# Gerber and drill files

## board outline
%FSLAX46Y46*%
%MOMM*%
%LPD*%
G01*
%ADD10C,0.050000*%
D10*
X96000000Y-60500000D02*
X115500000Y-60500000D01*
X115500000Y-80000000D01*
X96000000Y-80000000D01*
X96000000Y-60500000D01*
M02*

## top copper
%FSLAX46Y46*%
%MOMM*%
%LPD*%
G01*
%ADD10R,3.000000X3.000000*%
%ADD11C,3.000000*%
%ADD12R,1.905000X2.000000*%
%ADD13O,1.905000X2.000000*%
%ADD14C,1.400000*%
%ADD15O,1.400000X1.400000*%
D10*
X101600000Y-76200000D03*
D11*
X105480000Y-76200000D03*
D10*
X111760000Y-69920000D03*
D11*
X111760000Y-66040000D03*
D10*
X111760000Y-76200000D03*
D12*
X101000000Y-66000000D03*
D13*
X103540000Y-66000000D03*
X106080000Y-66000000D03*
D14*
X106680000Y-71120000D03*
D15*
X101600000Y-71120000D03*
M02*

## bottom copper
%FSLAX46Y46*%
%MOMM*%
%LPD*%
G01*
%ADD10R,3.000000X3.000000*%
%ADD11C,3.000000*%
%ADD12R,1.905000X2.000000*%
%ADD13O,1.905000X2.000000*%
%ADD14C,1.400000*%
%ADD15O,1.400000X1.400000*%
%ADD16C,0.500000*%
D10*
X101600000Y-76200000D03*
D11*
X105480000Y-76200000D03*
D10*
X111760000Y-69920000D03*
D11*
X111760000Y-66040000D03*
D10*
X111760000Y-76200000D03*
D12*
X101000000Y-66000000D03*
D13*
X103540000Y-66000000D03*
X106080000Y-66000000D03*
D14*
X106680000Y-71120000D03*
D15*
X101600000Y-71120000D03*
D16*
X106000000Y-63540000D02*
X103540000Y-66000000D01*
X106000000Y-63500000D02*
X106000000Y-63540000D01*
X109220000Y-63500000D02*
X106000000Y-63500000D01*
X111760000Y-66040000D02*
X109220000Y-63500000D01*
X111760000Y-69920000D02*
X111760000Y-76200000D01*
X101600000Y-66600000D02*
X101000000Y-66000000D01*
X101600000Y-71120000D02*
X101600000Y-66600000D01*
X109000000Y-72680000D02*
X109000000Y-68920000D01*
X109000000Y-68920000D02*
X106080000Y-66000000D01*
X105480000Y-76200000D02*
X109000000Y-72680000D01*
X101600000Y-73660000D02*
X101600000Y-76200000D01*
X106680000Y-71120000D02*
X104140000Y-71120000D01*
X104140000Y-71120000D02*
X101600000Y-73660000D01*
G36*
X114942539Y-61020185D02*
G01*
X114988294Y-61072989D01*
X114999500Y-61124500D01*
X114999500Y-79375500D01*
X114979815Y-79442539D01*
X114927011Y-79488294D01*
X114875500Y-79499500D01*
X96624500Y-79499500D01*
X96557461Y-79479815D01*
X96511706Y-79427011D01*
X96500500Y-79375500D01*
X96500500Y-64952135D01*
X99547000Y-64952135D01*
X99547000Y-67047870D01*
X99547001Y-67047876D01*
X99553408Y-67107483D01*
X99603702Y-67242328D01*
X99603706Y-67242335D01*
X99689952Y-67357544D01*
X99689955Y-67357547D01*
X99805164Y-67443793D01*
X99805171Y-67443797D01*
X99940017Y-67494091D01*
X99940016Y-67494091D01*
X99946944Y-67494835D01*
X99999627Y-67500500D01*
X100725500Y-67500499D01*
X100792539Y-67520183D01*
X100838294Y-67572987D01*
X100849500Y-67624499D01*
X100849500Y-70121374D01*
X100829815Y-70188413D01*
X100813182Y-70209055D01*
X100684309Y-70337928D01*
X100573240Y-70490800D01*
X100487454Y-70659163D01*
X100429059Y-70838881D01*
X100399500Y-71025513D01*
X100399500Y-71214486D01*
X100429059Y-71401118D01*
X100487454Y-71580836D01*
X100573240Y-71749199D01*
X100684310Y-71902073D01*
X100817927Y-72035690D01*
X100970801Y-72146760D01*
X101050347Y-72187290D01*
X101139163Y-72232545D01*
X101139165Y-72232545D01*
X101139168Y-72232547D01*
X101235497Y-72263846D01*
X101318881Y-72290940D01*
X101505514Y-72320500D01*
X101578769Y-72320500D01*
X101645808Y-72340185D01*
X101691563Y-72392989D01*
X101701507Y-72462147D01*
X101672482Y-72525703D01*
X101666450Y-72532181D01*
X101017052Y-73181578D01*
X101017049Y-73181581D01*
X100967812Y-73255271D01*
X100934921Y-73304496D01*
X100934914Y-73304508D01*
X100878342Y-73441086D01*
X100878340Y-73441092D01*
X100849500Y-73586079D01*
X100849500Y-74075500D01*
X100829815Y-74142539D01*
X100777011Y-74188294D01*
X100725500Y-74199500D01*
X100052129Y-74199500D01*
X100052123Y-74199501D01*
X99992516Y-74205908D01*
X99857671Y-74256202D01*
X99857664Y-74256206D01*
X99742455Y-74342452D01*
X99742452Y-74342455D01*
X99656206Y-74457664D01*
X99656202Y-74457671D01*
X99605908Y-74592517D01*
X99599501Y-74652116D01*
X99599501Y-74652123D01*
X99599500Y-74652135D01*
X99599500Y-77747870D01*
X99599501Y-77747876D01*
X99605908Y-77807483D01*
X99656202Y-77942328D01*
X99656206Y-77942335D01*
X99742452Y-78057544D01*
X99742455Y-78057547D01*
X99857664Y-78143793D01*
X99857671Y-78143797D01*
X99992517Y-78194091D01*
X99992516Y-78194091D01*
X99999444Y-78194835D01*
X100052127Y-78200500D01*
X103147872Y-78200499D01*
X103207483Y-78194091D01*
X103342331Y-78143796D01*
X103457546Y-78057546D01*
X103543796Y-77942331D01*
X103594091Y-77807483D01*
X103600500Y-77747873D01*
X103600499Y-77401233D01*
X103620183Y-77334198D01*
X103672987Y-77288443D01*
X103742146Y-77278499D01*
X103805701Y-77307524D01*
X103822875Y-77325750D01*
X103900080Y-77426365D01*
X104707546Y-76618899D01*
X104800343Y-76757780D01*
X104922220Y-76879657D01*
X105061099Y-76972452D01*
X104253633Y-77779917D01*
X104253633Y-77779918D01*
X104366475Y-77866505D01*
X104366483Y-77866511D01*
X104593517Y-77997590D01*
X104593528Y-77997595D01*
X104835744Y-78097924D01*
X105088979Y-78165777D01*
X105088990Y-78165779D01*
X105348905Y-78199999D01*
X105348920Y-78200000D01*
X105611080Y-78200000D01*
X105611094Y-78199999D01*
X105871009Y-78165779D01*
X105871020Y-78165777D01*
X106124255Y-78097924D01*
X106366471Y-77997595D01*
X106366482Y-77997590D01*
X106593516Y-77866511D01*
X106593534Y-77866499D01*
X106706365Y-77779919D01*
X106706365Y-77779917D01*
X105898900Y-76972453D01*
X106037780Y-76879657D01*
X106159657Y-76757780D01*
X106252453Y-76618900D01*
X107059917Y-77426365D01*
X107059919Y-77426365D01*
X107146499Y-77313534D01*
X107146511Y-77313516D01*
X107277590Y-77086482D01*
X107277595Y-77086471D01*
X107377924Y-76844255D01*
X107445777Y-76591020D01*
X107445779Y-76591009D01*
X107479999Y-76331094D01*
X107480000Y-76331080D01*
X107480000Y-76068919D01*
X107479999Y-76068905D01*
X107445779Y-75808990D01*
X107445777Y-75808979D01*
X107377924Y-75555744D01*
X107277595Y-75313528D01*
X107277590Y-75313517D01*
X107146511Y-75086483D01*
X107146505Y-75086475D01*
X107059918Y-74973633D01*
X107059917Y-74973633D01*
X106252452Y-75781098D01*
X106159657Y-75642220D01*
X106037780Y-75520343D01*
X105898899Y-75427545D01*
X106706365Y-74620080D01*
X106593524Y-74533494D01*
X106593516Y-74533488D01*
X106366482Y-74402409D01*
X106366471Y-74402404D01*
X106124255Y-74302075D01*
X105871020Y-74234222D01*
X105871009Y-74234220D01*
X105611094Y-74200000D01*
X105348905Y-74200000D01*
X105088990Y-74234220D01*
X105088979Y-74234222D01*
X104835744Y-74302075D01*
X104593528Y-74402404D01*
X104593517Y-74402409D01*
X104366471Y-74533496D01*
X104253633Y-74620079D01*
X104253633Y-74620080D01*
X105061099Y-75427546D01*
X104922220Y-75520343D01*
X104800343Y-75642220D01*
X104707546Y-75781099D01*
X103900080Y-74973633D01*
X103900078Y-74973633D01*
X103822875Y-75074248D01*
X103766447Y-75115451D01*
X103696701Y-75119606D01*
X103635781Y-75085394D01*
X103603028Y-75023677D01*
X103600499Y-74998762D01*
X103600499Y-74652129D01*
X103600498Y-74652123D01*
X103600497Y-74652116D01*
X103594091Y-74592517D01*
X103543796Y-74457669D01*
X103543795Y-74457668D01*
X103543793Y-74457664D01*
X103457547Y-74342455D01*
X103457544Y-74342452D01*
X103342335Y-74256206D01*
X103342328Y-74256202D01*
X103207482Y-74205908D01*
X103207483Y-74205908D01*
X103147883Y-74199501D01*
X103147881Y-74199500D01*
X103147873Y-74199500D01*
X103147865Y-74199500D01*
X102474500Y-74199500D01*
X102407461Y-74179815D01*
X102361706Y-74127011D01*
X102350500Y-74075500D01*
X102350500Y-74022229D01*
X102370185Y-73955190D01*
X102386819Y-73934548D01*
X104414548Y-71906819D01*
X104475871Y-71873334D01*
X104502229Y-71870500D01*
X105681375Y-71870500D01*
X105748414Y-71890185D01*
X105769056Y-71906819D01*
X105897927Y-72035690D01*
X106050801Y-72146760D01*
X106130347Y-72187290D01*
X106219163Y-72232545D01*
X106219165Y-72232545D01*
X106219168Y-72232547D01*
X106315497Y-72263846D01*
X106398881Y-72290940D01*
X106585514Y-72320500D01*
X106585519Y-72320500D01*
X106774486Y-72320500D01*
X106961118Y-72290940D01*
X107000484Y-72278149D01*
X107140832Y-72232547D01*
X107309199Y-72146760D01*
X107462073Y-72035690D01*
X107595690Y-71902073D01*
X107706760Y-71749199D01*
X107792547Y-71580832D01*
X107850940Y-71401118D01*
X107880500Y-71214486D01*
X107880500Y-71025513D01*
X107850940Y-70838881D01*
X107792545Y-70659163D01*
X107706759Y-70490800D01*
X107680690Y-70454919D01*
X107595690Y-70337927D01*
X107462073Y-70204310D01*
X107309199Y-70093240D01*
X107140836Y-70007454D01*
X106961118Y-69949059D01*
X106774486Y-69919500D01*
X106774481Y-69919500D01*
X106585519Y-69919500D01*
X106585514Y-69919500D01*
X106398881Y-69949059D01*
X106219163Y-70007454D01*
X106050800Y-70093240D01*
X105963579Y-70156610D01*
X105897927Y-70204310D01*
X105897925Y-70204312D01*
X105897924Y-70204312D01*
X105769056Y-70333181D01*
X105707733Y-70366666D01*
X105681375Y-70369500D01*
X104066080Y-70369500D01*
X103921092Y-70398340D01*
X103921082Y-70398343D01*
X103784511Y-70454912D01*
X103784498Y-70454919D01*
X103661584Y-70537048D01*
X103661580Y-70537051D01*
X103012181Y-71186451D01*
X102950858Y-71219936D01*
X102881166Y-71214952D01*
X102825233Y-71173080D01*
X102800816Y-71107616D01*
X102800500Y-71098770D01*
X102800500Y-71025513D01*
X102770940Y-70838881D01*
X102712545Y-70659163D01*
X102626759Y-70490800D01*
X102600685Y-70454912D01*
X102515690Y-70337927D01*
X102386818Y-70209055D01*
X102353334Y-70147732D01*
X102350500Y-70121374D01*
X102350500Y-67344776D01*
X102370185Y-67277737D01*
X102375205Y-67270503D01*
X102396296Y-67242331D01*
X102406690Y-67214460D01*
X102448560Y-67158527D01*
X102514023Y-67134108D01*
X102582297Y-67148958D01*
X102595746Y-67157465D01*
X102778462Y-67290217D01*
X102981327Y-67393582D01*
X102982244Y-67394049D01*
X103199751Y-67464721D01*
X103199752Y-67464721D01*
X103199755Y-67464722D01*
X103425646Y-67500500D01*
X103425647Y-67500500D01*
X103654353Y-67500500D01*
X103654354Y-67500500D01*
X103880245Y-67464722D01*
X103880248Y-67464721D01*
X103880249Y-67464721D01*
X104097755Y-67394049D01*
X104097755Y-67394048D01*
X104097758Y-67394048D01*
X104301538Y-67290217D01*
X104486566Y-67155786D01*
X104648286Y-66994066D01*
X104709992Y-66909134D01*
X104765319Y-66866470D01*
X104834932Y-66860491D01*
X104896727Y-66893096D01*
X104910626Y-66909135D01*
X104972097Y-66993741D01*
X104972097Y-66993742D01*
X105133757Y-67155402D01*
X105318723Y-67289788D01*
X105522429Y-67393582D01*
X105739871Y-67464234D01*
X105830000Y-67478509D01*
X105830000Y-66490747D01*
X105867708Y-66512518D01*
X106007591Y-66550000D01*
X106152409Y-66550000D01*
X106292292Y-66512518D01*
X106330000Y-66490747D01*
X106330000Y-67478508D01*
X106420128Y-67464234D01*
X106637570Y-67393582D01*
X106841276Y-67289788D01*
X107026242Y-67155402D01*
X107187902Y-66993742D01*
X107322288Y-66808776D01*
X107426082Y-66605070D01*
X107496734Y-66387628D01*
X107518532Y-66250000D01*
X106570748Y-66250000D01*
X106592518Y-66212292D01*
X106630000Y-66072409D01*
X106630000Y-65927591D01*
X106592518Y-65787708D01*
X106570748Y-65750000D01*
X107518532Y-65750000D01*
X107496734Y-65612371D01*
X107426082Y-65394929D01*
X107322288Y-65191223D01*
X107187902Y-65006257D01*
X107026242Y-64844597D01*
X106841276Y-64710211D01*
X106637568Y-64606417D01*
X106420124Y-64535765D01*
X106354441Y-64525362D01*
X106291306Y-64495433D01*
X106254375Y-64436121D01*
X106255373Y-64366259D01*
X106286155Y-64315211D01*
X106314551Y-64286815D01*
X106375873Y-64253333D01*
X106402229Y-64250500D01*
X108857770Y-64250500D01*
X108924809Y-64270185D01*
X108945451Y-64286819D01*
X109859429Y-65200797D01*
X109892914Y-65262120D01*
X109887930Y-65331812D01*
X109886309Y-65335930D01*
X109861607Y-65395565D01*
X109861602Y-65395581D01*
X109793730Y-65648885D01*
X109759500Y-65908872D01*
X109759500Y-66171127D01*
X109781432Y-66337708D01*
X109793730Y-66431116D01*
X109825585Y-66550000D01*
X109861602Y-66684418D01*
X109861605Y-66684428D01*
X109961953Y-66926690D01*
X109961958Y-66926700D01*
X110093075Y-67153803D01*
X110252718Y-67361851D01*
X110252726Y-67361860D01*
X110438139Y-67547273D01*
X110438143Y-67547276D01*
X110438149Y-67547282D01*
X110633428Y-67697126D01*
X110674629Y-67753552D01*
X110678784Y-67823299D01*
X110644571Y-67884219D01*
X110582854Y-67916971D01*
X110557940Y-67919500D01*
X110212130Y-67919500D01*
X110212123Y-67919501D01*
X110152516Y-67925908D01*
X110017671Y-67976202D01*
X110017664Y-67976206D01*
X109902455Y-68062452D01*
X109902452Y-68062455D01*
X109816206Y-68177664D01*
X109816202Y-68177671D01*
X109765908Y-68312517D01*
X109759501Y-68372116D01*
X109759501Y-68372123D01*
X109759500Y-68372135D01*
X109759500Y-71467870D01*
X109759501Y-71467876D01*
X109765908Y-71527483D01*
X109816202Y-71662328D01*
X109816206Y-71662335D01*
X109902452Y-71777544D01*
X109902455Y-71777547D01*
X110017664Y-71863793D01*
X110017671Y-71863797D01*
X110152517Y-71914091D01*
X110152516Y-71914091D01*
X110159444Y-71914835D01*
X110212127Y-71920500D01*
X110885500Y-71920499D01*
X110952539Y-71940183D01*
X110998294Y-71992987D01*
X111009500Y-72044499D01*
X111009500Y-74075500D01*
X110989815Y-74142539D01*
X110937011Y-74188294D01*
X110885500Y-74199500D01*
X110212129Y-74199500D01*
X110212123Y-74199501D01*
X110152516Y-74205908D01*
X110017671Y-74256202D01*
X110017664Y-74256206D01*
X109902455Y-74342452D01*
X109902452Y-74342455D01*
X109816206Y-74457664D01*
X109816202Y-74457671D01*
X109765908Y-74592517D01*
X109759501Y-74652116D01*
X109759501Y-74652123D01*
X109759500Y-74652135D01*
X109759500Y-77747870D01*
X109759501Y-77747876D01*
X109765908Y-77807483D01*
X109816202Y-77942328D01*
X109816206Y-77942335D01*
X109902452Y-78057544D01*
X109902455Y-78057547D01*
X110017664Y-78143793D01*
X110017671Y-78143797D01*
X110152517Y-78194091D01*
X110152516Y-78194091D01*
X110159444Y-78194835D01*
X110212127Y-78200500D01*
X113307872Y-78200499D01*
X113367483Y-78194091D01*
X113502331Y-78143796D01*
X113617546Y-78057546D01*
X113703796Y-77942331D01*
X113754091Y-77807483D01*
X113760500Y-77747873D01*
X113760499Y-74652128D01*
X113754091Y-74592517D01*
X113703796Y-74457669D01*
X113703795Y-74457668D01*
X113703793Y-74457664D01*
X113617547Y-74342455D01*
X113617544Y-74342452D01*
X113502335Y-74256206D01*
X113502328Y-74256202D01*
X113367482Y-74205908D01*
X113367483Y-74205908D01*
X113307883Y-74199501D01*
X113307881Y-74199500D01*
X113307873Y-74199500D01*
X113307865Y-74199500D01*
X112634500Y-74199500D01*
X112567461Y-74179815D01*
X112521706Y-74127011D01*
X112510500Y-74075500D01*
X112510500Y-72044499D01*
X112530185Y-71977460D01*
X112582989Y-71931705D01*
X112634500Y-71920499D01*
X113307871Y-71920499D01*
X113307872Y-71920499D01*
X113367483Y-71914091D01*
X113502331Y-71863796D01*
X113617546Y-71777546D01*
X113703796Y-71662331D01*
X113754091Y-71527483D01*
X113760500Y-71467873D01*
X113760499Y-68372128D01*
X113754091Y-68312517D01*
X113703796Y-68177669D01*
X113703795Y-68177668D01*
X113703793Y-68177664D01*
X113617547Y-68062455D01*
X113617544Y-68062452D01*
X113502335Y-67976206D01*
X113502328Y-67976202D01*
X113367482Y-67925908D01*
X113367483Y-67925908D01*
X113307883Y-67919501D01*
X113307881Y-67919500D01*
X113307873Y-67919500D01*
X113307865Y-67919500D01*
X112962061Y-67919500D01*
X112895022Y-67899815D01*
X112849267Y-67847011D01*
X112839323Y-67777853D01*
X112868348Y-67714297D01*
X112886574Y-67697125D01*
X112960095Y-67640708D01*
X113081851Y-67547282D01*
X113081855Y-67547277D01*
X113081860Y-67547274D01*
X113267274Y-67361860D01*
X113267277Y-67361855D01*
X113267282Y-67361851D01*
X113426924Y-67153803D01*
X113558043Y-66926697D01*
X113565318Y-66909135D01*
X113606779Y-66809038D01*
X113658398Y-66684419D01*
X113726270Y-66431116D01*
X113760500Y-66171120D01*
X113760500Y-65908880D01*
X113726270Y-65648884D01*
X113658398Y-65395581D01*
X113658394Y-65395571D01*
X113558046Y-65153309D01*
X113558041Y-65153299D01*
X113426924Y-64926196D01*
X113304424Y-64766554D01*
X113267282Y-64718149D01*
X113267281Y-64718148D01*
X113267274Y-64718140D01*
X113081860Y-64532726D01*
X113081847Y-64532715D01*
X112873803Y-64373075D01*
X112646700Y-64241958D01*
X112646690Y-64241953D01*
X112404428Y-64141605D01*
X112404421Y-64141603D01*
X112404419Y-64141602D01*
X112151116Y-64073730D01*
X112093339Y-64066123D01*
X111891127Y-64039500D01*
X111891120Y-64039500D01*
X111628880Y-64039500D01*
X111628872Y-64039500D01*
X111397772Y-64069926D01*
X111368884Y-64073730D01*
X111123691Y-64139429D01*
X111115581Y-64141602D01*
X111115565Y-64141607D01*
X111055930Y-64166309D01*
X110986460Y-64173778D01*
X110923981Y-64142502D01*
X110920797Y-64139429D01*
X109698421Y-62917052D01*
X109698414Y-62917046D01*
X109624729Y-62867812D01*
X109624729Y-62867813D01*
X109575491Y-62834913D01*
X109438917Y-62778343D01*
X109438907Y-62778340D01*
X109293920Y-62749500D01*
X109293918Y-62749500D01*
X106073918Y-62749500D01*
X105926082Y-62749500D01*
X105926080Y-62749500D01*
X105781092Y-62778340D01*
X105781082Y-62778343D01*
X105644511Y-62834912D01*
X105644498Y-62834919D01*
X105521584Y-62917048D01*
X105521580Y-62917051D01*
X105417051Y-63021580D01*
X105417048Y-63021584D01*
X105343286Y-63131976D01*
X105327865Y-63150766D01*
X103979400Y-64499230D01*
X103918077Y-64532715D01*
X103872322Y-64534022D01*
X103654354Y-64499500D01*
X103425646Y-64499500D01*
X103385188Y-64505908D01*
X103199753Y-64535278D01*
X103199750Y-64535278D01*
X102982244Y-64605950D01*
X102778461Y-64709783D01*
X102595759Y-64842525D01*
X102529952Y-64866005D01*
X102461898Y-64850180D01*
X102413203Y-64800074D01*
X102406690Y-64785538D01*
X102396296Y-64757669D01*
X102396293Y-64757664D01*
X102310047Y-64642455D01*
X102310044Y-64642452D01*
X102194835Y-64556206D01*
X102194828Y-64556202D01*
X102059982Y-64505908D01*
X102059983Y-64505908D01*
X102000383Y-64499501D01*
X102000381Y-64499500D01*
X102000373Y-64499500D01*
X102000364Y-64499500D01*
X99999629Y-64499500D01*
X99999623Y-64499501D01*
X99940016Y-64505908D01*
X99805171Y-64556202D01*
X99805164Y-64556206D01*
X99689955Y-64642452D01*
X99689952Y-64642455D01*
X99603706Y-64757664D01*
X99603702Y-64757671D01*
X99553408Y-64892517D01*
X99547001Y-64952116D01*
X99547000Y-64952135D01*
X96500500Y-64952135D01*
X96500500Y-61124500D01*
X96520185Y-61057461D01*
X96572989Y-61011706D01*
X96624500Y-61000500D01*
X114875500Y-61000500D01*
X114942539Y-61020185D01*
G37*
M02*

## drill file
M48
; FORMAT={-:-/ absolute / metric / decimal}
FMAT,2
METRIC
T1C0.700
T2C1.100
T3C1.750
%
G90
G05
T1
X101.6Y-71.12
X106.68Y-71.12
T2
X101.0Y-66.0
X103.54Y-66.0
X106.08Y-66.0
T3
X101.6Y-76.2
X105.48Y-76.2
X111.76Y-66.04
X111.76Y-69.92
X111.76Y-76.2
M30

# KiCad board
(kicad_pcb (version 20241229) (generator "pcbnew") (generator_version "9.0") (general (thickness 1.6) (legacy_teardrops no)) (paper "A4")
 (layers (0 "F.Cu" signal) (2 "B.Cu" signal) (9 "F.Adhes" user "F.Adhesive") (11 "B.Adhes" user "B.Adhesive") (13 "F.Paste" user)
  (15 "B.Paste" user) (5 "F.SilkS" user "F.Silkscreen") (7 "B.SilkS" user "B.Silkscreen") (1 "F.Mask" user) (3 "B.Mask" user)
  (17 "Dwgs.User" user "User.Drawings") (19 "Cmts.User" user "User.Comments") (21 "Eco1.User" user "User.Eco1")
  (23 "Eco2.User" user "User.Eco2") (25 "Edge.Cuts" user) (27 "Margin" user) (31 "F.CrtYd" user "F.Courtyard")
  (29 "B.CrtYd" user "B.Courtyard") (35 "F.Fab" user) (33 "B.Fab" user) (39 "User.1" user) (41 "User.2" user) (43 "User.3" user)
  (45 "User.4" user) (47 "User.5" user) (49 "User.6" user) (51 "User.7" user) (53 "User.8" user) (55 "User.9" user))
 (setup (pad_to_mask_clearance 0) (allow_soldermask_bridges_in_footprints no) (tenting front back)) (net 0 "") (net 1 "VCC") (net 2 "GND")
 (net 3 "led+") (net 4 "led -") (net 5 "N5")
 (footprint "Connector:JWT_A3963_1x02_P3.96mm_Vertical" (layer "F.Cu") (at 101.6 76.2)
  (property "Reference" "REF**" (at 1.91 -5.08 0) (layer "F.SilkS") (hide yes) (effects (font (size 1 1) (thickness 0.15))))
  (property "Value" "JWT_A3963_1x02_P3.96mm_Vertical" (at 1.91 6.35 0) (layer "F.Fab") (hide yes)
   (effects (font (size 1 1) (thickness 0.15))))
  (pad "1" thru_hole rect (at 0 0) (size 3 3) (drill 1.75) (layers "*.Cu" "*.Mask") (remove_unused_layers no) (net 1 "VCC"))
  (pad "2" thru_hole circle (at 3.88 0) (size 3 3) (drill 1.75) (layers "*.Cu" "*.Mask") (remove_unused_layers no) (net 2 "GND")))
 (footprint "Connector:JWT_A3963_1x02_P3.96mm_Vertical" (layer "F.Cu") (at 111.76 69.92 90)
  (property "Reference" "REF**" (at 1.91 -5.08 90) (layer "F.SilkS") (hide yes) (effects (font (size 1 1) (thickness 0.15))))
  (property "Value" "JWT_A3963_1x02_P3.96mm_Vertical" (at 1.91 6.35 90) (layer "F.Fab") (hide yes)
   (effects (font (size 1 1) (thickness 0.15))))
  (pad "1" thru_hole rect (at 0 0 90) (size 3 3) (drill 1.75) (layers "*.Cu" "*.Mask") (remove_unused_layers no) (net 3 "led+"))
  (pad "2" thru_hole circle (at 3.88 0 90) (size 3 3) (drill 1.75) (layers "*.Cu" "*.Mask") (remove_unused_layers no) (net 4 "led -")))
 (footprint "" (layer "F.Cu") (at 111.76 76.2)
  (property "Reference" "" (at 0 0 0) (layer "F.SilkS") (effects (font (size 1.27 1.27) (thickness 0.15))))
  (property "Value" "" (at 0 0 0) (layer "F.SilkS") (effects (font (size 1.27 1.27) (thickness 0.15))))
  (pad "1" thru_hole rect (at 0 0 90) (size 3 3) (drill 1.75) (layers "*.Cu" "*.Mask") (remove_unused_layers no) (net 3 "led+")))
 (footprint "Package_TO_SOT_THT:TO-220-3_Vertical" (layer "F.Cu") (at 101 66)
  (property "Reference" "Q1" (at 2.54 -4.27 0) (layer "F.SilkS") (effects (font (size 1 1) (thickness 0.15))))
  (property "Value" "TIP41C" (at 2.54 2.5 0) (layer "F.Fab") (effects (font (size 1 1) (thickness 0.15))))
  (pad "1" thru_hole rect (at 0 0) (size 1.905 2) (drill 1.1) (layers "*.Cu" "*.Mask") (remove_unused_layers no) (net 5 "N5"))
  (pad "2" thru_hole oval (at 2.54 0) (size 1.905 2) (drill 1.1) (layers "*.Cu" "*.Mask") (remove_unused_layers no) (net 4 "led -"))
  (pad "3" thru_hole oval (at 5.08 0) (size 1.905 2) (drill 1.1) (layers "*.Cu" "*.Mask") (remove_unused_layers no) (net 2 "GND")))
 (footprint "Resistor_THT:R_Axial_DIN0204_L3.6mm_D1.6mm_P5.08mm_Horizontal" (layer "F.Cu") (at 106.68 71.12 180)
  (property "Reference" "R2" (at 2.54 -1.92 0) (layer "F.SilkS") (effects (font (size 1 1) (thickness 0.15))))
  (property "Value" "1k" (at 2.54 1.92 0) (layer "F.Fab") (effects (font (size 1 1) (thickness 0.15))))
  (pad "1" thru_hole circle (at 0 0 180) (size 1.4 1.4) (drill 0.7) (layers "*.Cu" "*.Mask") (remove_unused_layers no) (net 1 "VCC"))
  (pad "2" thru_hole oval (at 5.08 0 180) (size 1.4 1.4) (drill 0.7) (layers "*.Cu" "*.Mask") (remove_unused_layers no) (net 5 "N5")))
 (gr_rect (start 96 60.5) (end 115.5 80) (stroke (width 0.05) (type default)) (fill no) (layer "Edge.Cuts"))
 (segment (start 106 63.54) (end 103.54 66) (width 0.5) (layer "B.Cu") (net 4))
 (segment (start 106 63.5) (end 106 63.54) (width 0.5) (layer "B.Cu") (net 4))
 (segment (start 109.22 63.5) (end 106 63.5) (width 0.5) (layer "B.Cu") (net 4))
 (segment (start 111.76 66.04) (end 109.22 63.5) (width 0.5) (layer "B.Cu") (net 4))
 (segment (start 111.76 69.92) (end 111.76 76.2) (width 0.5) (layer "B.Cu") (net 3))
 (segment (start 101.6 66.6) (end 101 66) (width 0.5) (layer "B.Cu") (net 5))
 (segment (start 101.6 71.12) (end 101.6 66.6) (width 0.5) (layer "B.Cu") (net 5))
 (segment (start 109 72.68) (end 109 68.92) (width 0.5) (layer "B.Cu") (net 2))
 (segment (start 109 68.92) (end 106.08 66) (width 0.5) (layer "B.Cu") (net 2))
 (segment (start 105.48 76.2) (end 109 72.68) (width 0.5) (layer "B.Cu") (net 2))
 (segment (start 101.6 73.66) (end 101.6 76.2) (width 0.5) (layer "B.Cu") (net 1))
 (segment (start 106.68 71.12) (end 104.14 71.12) (width 0.5) (layer "B.Cu") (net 1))
 (segment (start 104.14 71.12) (end 101.6 73.66) (width 0.5) (layer "B.Cu") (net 1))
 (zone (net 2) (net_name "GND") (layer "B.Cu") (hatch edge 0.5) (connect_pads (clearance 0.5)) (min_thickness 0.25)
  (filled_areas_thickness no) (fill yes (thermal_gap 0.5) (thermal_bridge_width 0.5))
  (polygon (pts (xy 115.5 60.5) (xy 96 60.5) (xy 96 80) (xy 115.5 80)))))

